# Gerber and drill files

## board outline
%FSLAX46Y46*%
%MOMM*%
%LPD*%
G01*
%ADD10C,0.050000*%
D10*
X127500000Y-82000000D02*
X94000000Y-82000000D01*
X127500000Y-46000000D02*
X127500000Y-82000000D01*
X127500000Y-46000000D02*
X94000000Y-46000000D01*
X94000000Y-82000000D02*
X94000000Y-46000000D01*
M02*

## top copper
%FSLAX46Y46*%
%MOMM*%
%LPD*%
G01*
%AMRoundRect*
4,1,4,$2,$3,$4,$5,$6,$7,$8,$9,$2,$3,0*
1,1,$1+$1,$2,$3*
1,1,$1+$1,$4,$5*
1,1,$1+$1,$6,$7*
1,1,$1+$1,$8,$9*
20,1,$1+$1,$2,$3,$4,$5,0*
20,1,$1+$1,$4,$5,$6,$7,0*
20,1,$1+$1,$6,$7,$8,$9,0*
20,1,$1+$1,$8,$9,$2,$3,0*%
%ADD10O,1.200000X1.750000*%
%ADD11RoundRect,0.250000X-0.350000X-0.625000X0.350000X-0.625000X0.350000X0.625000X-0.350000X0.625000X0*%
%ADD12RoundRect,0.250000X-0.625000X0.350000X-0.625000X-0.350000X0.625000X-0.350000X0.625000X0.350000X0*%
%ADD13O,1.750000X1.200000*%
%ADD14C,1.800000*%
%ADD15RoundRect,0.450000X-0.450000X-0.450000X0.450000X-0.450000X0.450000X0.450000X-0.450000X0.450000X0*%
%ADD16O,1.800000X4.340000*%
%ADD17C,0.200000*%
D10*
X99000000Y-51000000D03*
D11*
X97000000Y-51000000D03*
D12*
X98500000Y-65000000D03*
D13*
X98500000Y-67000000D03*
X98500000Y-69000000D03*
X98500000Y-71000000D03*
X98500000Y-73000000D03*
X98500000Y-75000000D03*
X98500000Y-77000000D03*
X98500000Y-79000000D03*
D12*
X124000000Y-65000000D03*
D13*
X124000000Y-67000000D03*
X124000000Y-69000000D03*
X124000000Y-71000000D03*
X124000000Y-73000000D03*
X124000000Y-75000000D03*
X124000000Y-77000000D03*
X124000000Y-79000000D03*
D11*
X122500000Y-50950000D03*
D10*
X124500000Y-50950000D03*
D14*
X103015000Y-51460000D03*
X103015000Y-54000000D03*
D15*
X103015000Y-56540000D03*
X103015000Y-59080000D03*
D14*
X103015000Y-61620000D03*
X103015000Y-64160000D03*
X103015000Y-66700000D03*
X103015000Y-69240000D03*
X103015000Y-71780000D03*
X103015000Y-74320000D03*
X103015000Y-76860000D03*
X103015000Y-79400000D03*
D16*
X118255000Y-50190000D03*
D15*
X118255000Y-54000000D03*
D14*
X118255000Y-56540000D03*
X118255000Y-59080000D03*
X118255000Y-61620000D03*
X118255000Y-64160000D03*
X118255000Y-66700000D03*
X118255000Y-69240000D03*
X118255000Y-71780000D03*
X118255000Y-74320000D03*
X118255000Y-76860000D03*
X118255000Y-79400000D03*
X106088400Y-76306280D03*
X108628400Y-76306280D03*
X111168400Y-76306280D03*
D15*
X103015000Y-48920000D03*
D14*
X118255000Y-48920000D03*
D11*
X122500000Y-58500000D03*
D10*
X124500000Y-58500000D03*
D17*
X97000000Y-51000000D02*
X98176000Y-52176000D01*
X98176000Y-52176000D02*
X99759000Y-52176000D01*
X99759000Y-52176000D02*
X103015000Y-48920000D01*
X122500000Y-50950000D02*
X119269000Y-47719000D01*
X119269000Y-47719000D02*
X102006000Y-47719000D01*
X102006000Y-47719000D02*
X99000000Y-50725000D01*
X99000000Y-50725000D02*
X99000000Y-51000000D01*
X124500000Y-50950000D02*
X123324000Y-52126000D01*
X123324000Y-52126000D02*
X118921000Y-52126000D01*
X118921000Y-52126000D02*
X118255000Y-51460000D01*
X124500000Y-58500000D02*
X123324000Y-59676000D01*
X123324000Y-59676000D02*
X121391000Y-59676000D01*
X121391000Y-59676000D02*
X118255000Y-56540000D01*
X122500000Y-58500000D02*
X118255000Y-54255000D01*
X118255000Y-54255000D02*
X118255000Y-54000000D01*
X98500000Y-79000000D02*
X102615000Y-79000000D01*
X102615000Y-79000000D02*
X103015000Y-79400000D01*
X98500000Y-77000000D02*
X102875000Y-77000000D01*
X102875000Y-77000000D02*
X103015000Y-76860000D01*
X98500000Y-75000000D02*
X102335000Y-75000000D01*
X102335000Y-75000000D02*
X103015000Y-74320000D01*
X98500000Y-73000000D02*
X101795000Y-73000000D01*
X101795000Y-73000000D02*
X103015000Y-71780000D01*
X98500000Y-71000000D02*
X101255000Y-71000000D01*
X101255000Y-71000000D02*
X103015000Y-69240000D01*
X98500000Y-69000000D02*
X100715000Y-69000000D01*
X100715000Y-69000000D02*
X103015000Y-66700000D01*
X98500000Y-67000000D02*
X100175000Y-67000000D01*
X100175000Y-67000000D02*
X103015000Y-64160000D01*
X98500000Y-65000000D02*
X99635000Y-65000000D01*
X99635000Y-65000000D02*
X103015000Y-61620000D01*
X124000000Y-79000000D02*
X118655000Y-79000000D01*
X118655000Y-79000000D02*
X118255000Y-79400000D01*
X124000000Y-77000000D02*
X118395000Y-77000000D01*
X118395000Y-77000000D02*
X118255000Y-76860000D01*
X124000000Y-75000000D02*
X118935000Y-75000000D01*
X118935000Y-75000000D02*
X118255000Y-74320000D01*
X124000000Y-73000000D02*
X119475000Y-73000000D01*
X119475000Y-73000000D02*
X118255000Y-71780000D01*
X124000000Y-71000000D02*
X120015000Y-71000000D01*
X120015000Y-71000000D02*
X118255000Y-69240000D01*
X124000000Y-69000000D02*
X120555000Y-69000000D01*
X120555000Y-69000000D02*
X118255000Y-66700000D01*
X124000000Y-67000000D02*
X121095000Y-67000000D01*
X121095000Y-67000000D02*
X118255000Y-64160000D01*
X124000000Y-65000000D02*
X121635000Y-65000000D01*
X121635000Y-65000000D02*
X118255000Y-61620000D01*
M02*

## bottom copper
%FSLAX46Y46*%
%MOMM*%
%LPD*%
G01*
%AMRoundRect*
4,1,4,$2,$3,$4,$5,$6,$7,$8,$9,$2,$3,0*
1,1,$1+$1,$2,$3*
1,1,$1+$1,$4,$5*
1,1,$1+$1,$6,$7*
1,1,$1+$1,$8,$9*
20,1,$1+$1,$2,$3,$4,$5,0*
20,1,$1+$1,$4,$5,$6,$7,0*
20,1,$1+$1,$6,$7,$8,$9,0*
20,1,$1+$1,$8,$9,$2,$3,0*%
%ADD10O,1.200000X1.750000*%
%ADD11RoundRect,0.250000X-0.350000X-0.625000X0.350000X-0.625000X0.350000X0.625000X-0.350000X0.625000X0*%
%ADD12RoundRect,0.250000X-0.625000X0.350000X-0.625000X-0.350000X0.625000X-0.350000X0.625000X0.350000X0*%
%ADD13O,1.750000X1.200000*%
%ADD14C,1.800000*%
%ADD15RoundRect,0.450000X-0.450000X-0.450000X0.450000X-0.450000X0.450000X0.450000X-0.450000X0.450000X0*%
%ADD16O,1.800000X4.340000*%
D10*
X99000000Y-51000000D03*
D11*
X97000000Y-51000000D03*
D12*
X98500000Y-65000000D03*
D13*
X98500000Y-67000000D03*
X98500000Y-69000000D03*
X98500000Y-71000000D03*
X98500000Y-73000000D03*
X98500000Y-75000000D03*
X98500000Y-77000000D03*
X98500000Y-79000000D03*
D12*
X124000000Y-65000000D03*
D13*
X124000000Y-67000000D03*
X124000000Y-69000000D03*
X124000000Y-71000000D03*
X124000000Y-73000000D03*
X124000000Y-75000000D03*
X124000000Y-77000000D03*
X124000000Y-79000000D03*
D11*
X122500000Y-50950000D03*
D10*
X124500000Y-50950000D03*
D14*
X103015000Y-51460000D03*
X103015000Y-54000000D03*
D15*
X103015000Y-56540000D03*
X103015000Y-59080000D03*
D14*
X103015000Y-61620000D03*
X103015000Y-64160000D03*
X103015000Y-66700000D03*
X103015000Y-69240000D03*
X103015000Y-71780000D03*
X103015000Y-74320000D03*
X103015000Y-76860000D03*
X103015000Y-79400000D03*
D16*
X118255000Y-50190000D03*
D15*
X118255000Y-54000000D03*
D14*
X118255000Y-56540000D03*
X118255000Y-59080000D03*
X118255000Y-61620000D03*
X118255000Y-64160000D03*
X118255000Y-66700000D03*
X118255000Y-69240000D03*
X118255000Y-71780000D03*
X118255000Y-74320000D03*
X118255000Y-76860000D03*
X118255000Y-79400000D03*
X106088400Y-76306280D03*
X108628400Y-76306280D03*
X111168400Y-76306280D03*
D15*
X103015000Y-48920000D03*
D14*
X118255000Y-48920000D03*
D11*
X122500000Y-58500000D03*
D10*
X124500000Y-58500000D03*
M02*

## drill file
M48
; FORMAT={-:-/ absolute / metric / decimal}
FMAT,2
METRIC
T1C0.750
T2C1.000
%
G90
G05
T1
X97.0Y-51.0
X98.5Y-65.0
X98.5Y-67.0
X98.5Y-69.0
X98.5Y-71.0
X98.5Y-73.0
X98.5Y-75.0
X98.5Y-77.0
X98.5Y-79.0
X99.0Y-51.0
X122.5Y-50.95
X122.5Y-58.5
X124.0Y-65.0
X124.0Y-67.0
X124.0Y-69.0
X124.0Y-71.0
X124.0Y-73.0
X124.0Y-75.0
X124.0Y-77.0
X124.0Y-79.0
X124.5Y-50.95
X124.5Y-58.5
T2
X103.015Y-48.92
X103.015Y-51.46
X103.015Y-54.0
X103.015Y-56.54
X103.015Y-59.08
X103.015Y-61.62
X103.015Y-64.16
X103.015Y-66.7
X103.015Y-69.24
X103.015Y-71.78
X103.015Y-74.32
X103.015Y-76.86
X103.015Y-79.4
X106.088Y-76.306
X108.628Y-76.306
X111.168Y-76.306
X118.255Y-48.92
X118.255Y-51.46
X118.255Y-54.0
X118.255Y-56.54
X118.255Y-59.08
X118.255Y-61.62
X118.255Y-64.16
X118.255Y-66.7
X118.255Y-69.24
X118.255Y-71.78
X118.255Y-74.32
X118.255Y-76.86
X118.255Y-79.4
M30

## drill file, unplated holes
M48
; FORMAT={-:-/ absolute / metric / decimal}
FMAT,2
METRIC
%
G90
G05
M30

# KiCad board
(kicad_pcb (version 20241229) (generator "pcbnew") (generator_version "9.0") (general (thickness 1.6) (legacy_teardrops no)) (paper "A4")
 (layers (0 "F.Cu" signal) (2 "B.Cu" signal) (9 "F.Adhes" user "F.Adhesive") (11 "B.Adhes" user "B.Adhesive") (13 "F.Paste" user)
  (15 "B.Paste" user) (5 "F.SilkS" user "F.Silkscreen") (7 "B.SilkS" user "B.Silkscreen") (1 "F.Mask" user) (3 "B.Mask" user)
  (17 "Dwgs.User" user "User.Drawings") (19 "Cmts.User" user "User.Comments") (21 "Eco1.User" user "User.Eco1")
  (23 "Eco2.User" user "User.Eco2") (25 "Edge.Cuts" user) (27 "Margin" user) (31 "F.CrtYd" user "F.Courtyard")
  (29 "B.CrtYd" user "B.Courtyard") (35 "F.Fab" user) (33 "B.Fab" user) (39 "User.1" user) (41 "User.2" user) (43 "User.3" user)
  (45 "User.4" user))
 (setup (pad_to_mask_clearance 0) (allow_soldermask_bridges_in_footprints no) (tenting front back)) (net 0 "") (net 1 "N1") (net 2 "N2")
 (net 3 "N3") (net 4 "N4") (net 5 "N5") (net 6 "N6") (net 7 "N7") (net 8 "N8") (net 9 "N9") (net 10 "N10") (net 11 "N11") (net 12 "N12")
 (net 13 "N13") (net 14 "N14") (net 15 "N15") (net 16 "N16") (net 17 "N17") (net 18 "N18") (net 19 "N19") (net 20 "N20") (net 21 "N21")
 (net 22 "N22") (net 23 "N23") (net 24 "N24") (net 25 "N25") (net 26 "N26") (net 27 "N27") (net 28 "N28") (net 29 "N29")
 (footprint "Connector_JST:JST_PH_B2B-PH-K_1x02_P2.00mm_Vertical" (layer "F.Cu") (at 97 51)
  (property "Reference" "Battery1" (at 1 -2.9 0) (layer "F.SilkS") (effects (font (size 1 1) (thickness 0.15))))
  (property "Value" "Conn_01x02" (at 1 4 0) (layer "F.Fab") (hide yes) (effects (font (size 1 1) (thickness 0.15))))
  (pad "1" thru_hole roundrect (at 0 0) (size 1.2 1.75) (drill 0.75) (layers "*.Cu" "*.Mask") (remove_unused_layers no)
   (roundrect_rratio 0.208333) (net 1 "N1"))
  (pad "2" thru_hole oval (at 2 0) (size 1.2 1.75) (drill 0.75) (layers "*.Cu" "*.Mask") (remove_unused_layers no) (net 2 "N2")))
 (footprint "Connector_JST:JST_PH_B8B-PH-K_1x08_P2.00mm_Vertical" (layer "F.Cu") (at 98.5 65 -90)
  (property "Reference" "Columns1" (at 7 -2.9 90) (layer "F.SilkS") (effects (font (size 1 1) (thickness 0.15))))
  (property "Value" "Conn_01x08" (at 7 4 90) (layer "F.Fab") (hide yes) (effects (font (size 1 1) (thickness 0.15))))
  (pad "1" thru_hole roundrect (at 0 0 270) (size 1.2 1.75) (drill 0.75) (layers "*.Cu" "*.Mask") (remove_unused_layers no)
   (roundrect_rratio 0.208333) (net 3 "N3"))
  (pad "2" thru_hole oval (at 2 0 270) (size 1.2 1.75) (drill 0.75) (layers "*.Cu" "*.Mask") (remove_unused_layers no) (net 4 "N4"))
  (pad "3" thru_hole oval (at 4 0 270) (size 1.2 1.75) (drill 0.75) (layers "*.Cu" "*.Mask") (remove_unused_layers no) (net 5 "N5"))
  (pad "4" thru_hole oval (at 6 0 270) (size 1.2 1.75) (drill 0.75) (layers "*.Cu" "*.Mask") (remove_unused_layers no) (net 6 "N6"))
  (pad "5" thru_hole oval (at 8 0 270) (size 1.2 1.75) (drill 0.75) (layers "*.Cu" "*.Mask") (remove_unused_layers no) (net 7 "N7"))
  (pad "6" thru_hole oval (at 10 0 270) (size 1.2 1.75) (drill 0.75) (layers "*.Cu" "*.Mask") (remove_unused_layers no) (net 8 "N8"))
  (pad "7" thru_hole oval (at 12 0 270) (size 1.2 1.75) (drill 0.75) (layers "*.Cu" "*.Mask") (remove_unused_layers no) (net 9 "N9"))
  (pad "8" thru_hole oval (at 14 0 270) (size 1.2 1.75) (drill 0.75) (layers "*.Cu" "*.Mask") (remove_unused_layers no) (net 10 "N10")))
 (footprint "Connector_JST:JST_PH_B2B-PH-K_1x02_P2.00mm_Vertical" (layer "F.Cu") (at 122.5 50.95)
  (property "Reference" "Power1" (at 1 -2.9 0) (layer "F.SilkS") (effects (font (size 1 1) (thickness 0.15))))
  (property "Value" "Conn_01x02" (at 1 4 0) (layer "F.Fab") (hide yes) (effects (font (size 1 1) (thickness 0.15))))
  (pad "1" thru_hole roundrect (at 0 0) (size 1.2 1.75) (drill 0.75) (layers "*.Cu" "*.Mask") (remove_unused_layers no)
   (roundrect_rratio 0.208333) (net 2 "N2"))
  (pad "2" thru_hole oval (at 2 0) (size 1.2 1.75) (drill 0.75) (layers "*.Cu" "*.Mask") (remove_unused_layers no) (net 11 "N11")))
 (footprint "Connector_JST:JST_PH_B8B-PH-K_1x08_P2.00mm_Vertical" (layer "F.Cu") (at 124 65 -90)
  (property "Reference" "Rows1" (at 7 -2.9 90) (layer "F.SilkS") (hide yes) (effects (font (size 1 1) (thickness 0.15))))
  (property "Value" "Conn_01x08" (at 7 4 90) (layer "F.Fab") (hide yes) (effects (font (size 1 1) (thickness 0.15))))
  (pad "1" thru_hole roundrect (at 0 0 270) (size 1.2 1.75) (drill 0.75) (layers "*.Cu" "*.Mask") (remove_unused_layers no)
   (roundrect_rratio 0.208333) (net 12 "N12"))
  (pad "2" thru_hole oval (at 2 0 270) (size 1.2 1.75) (drill 0.75) (layers "*.Cu" "*.Mask") (remove_unused_layers no) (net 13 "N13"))
  (pad "3" thru_hole oval (at 4 0 270) (size 1.2 1.75) (drill 0.75) (layers "*.Cu" "*.Mask") (remove_unused_layers no) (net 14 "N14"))
  (pad "4" thru_hole oval (at 6 0 270) (size 1.2 1.75) (drill 0.75) (layers "*.Cu" "*.Mask") (remove_unused_layers no) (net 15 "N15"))
  (pad "5" thru_hole oval (at 8 0 270) (size 1.2 1.75) (drill 0.75) (layers "*.Cu" "*.Mask") (remove_unused_layers no) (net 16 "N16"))
  (pad "6" thru_hole oval (at 10 0 270) (size 1.2 1.75) (drill 0.75) (layers "*.Cu" "*.Mask") (remove_unused_layers no) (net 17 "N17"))
  (pad "7" thru_hole oval (at 12 0 270) (size 1.2 1.75) (drill 0.75) (layers "*.Cu" "*.Mask") (remove_unused_layers no) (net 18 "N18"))
  (pad "8" thru_hole oval (at 14 0 270) (size 1.2 1.75) (drill 0.75) (layers "*.Cu" "*.Mask") (remove_unused_layers no) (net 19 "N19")))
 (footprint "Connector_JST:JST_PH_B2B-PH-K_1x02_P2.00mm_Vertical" (layer "F.Cu") (at 122.5 58.5)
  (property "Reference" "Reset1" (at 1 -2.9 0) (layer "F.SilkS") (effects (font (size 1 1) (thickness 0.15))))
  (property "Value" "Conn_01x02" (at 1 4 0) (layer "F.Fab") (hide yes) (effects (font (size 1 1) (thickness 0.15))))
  (pad "1" thru_hole roundrect (at 0 0) (size 1.2 1.75) (drill 0.75) (layers "*.Cu" "*.Mask") (remove_unused_layers no)
   (roundrect_rratio 0.208333) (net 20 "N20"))
  (pad "2" thru_hole oval (at 2 0) (size 1.2 1.75) (drill 0.75) (layers "*.Cu" "*.Mask") (remove_unused_layers no) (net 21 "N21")))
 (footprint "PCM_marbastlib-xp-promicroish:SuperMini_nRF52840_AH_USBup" (layer "F.Cu") (at 110.635 65.43)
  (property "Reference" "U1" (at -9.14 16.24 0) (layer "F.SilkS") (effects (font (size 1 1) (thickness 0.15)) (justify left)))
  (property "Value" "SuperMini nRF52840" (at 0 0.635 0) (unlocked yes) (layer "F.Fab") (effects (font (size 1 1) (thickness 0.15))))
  (pad "1" thru_hole circle (at -7.62 -13.97) (size 1.8 1.8) (drill 1) (layers "*.Cu" "B.Mask") (remove_unused_layers no) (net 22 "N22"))
  (pad "2" thru_hole circle (at -7.62 -11.43) (size 1.8 1.8) (drill 1) (layers "*.Cu" "B.Mask") (remove_unused_layers no) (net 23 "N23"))
  (pad "3" thru_hole roundrect (at -7.62 -8.89) (size 1.8 1.8) (drill 1) (layers "*.Cu" "B.Mask") (remove_unused_layers no)
   (roundrect_rratio 0.25) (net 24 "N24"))
  (pad "4" thru_hole roundrect (at -7.62 -6.35) (size 1.8 1.8) (drill 1) (layers "*.Cu" "B.Mask") (remove_unused_layers no)
   (roundrect_rratio 0.25) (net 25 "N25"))
  (pad "5" thru_hole circle (at -7.62 -3.81) (size 1.8 1.8) (drill 1) (layers "*.Cu" "B.Mask") (remove_unused_layers no) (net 3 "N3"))
  (pad "6" thru_hole circle (at -7.62 -1.27) (size 1.8 1.8) (drill 1) (layers "*.Cu" "B.Mask") (remove_unused_layers no) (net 4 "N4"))
  (pad "7" thru_hole circle (at -7.62 1.27) (size 1.8 1.8) (drill 1) (layers "*.Cu" "B.Mask") (remove_unused_layers no) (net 5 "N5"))
  (pad "8" thru_hole circle (at -7.62 3.81) (size 1.8 1.8) (drill 1) (layers "*.Cu" "B.Mask") (remove_unused_layers no) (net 6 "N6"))
  (pad "9" thru_hole circle (at -7.62 6.35) (size 1.8 1.8) (drill 1) (layers "*.Cu" "B.Mask") (remove_unused_layers no) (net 7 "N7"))
  (pad "10" thru_hole circle (at -7.62 8.89) (size 1.8 1.8) (drill 1) (layers "*.Cu" "B.Mask") (remove_unused_layers no) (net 8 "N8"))
  (pad "11" thru_hole circle (at -7.62 11.43) (size 1.8 1.8) (drill 1) (layers "*.Cu" "B.Mask") (remove_unused_layers no) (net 9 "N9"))
  (pad "12" thru_hole circle (at -7.62 13.97) (size 1.8 1.8) (drill 1) (layers "*.Cu" "B.Mask") (remove_unused_layers no) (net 10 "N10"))
  (pad "13" thru_hole oval (at 7.62 -13.97) (size 1.8 4.34) (drill 1 (offset 0 -1.27)) (layers "*.Cu" "B.Mask") (remove_unused_layers no)
   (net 11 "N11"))
  (pad "14" thru_hole roundrect (at 7.62 -11.43) (size 1.8 1.8) (drill 1) (layers "*.Cu" "B.Mask") (remove_unused_layers no)
   (roundrect_rratio 0.25) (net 20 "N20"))
  (pad "15" thru_hole circle (at 7.62 -8.89) (size 1.8 1.8) (drill 1) (layers "*.Cu" "B.Mask") (remove_unused_layers no) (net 21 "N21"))
  (pad "16" thru_hole circle (at 7.62 -6.35) (size 1.8 1.8) (drill 1) (layers "*.Cu" "B.Mask") (remove_unused_layers no) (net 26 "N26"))
  (pad "17" thru_hole circle (at 7.62 -3.81) (size 1.8 1.8) (drill 1) (layers "*.Cu" "B.Mask") (remove_unused_layers no) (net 12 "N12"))
  (pad "18" thru_hole circle (at 7.62 -1.27) (size 1.8 1.8) (drill 1) (layers "*.Cu" "B.Mask") (remove_unused_layers no) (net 13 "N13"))
  (pad "19" thru_hole circle (at 7.62 1.27) (size 1.8 1.8) (drill 1) (layers "*.Cu" "B.Mask") (remove_unused_layers no) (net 14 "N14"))
  (pad "20" thru_hole circle (at 7.62 3.81) (size 1.8 1.8) (drill 1) (layers "*.Cu" "B.Mask") (remove_unused_layers no) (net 15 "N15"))
  (pad "21" thru_hole circle (at 7.62 6.35) (size 1.8 1.8) (drill 1) (layers "*.Cu" "B.Mask") (remove_unused_layers no) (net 16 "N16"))
  (pad "22" thru_hole circle (at 7.62 8.89) (size 1.8 1.8) (drill 1) (layers "*.Cu" "B.Mask") (remove_unused_layers no) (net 17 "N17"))
  (pad "23" thru_hole circle (at 7.62 11.43) (size 1.8 1.8) (drill 1) (layers "*.Cu" "B.Mask") (remove_unused_layers no) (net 18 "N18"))
  (pad "24" thru_hole circle (at 7.62 13.97) (size 1.8 1.8) (drill 1) (layers "*.Cu" "B.Mask") (remove_unused_layers no) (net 19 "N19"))
  (pad "25" thru_hole circle (at -4.5466 10.87628) (size 1.8 1.8) (drill 1) (layers "*.Cu" "B.Mask") (remove_unused_layers no)
   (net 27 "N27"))
  (pad "26" thru_hole circle (at -2.0066 10.87628) (size 1.8 1.8) (drill 1) (layers "*.Cu" "B.Mask") (remove_unused_layers no)
   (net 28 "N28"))
  (pad "27" thru_hole circle (at 0.5334 10.87628) (size 1.8 1.8) (drill 1) (layers "*.Cu" "B.Mask") (remove_unused_layers no) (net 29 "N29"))
  (pad "28" thru_hole roundrect (at -7.62 -16.51) (size 1.8 1.8) (drill 1) (layers "*.Cu" "B.Mask") (remove_unused_layers no)
   (roundrect_rratio 0.25) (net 1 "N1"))
  (pad "29" thru_hole circle (at 7.62 -16.51) (size 1.8 1.8) (drill 1) (layers "*.Cu" "B.Mask") (remove_unused_layers no) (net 11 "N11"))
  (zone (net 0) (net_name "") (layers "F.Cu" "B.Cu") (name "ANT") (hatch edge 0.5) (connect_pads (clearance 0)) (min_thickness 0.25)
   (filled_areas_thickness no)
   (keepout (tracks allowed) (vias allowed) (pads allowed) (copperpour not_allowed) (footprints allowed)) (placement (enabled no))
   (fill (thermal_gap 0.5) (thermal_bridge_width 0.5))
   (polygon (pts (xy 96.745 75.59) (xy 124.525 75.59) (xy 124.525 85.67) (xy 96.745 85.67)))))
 (gr_line (start 127.5 46) (end 127.5 82) (stroke (width 0.05) (type default)) (layer "Edge.Cuts"))
 (gr_line (start 127.5 82) (end 94 82) (stroke (width 0.05) (type default)) (layer "Edge.Cuts"))
 (gr_line (start 127.5 46) (end 94 46) (stroke (width 0.05) (type default)) (layer "Edge.Cuts"))
 (gr_line (start 94 82) (end 94 46) (stroke (width 0.05) (type default)) (layer "Edge.Cuts"))
 (segment (start 99.759 52.176) (end 103.015 48.92) (width 0.2) (layer "F.Cu") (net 1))
 (segment (start 97 51) (end 98.176 52.176) (width 0.2) (layer "F.Cu") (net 1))
 (segment (start 98.176 52.176) (end 99.759 52.176) (width 0.2) (layer "F.Cu") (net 1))
 (segment (start 102.006 47.719) (end 99 50.725) (width 0.2) (layer "F.Cu") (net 2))
 (segment (start 119.269 47.719) (end 102.006 47.719) (width 0.2) (layer "F.Cu") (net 2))
 (segment (start 99 50.725) (end 99 51) (width 0.2) (layer "F.Cu") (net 2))
 (segment (start 122.5 50.95) (end 119.269 47.719) (width 0.2) (layer "F.Cu") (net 2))
 (segment (start 101.795 73) (end 103.015 71.78) (width 0.2) (layer "F.Cu") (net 7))
 (segment (start 98.5 73) (end 101.795 73) (width 0.2) (layer "F.Cu") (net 7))
 (segment (start 102.335 75) (end 103.015 74.32) (width 0.2) (layer "F.Cu") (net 8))
 (segment (start 98.5 75) (end 102.335 75) (width 0.2) (layer "F.Cu") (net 8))
 (segment (start 100.715 69) (end 103.015 66.7) (width 0.2) (layer "F.Cu") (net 5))
 (segment (start 98.5 69) (end 100.715 69) (width 0.2) (layer "F.Cu") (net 5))
 (segment (start 100.175 67) (end 103.015 64.16) (width 0.2) (layer "F.Cu") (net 4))
 (segment (start 98.5 67) (end 100.175 67) (width 0.2) (layer "F.Cu") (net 4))
 (segment (start 101.255 71) (end 103.015 69.24) (width 0.2) (layer "F.Cu") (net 6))
 (segment (start 98.5 71) (end 101.255 71) (width 0.2) (layer "F.Cu") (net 6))
 (segment (start 98.5 77) (end 102.875 77) (width 0.2) (layer "F.Cu") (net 9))
 (segment (start 102.875 77) (end 103.015 76.86) (width 0.2) (layer "F.Cu") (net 9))
 (segment (start 98.5 79) (end 102.615 79) (width 0.2) (layer "F.Cu") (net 10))
 (segment (start 102.615 79) (end 103.015 79.4) (width 0.2) (layer "F.Cu") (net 10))
 (segment (start 98.5 65) (end 99.635 65) (width 0.2) (layer "F.Cu") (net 3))
 (segment (start 99.635 65) (end 103.015 61.62) (width 0.2) (layer "F.Cu") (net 3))
 (segment (start 123.324 52.126) (end 118.921 52.126) (width 0.2) (layer "F.Cu") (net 11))
 (segment (start 118.921 52.126) (end 118.255 51.46) (width 0.2) (layer "F.Cu") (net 11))
 (segment (start 124.5 50.95) (end 123.324 52.126) (width 0.2) (layer "F.Cu") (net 11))
 (segment (start 123.324 59.676) (end 121.391 59.676) (width 0.2) (layer "F.Cu") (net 21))
 (segment (start 124.5 58.5) (end 123.324 59.676) (width 0.2) (layer "F.Cu") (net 21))
 (segment (start 121.391 59.676) (end 118.255 56.54) (width 0.2) (layer "F.Cu") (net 21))
 (segment (start 124 65) (end 121.635 65) (width 0.2) (layer "F.Cu") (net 12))
 (segment (start 121.635 65) (end 118.255 61.62) (width 0.2) (layer "F.Cu") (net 12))
 (segment (start 124 71) (end 120.015 71) (width 0.2) (layer "F.Cu") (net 15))
 (segment (start 120.015 71) (end 118.255 69.24) (width 0.2) (layer "F.Cu") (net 15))
 (segment (start 124 67) (end 121.095 67) (width 0.2) (layer "F.Cu") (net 13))
 (segment (start 121.095 67) (end 118.255 64.16) (width 0.2) (layer "F.Cu") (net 13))
 (segment (start 124 77) (end 118.395 77) (width 0.2) (layer "F.Cu") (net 18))
 (segment (start 118.395 77) (end 118.255 76.86) (width 0.2) (layer "F.Cu") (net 18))
 (segment (start 120.555 69) (end 118.255 66.7) (width 0.2) (layer "F.Cu") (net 14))
 (segment (start 124 69) (end 120.555 69) (width 0.2) (layer "F.Cu") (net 14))
 (segment (start 124 75) (end 118.935 75) (width 0.2) (layer "F.Cu") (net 17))
 (segment (start 118.935 75) (end 118.255 74.32) (width 0.2) (layer "F.Cu") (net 17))
 (segment (start 118.655 79) (end 118.255 79.4) (width 0.2) (layer "F.Cu") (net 19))
 (segment (start 124 79) (end 118.655 79) (width 0.2) (layer "F.Cu") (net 19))
 (segment (start 124 73) (end 119.475 73) (width 0.2) (layer "F.Cu") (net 16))
 (segment (start 119.475 73) (end 118.255 71.78) (width 0.2) (layer "F.Cu") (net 16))
 (segment (start 122.5 58.5) (end 118.255 54.255) (width 0.2) (layer "F.Cu") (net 20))
 (segment (start 118.255 54.255) (end 118.255 54) (width 0.2) (layer "F.Cu") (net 20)))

